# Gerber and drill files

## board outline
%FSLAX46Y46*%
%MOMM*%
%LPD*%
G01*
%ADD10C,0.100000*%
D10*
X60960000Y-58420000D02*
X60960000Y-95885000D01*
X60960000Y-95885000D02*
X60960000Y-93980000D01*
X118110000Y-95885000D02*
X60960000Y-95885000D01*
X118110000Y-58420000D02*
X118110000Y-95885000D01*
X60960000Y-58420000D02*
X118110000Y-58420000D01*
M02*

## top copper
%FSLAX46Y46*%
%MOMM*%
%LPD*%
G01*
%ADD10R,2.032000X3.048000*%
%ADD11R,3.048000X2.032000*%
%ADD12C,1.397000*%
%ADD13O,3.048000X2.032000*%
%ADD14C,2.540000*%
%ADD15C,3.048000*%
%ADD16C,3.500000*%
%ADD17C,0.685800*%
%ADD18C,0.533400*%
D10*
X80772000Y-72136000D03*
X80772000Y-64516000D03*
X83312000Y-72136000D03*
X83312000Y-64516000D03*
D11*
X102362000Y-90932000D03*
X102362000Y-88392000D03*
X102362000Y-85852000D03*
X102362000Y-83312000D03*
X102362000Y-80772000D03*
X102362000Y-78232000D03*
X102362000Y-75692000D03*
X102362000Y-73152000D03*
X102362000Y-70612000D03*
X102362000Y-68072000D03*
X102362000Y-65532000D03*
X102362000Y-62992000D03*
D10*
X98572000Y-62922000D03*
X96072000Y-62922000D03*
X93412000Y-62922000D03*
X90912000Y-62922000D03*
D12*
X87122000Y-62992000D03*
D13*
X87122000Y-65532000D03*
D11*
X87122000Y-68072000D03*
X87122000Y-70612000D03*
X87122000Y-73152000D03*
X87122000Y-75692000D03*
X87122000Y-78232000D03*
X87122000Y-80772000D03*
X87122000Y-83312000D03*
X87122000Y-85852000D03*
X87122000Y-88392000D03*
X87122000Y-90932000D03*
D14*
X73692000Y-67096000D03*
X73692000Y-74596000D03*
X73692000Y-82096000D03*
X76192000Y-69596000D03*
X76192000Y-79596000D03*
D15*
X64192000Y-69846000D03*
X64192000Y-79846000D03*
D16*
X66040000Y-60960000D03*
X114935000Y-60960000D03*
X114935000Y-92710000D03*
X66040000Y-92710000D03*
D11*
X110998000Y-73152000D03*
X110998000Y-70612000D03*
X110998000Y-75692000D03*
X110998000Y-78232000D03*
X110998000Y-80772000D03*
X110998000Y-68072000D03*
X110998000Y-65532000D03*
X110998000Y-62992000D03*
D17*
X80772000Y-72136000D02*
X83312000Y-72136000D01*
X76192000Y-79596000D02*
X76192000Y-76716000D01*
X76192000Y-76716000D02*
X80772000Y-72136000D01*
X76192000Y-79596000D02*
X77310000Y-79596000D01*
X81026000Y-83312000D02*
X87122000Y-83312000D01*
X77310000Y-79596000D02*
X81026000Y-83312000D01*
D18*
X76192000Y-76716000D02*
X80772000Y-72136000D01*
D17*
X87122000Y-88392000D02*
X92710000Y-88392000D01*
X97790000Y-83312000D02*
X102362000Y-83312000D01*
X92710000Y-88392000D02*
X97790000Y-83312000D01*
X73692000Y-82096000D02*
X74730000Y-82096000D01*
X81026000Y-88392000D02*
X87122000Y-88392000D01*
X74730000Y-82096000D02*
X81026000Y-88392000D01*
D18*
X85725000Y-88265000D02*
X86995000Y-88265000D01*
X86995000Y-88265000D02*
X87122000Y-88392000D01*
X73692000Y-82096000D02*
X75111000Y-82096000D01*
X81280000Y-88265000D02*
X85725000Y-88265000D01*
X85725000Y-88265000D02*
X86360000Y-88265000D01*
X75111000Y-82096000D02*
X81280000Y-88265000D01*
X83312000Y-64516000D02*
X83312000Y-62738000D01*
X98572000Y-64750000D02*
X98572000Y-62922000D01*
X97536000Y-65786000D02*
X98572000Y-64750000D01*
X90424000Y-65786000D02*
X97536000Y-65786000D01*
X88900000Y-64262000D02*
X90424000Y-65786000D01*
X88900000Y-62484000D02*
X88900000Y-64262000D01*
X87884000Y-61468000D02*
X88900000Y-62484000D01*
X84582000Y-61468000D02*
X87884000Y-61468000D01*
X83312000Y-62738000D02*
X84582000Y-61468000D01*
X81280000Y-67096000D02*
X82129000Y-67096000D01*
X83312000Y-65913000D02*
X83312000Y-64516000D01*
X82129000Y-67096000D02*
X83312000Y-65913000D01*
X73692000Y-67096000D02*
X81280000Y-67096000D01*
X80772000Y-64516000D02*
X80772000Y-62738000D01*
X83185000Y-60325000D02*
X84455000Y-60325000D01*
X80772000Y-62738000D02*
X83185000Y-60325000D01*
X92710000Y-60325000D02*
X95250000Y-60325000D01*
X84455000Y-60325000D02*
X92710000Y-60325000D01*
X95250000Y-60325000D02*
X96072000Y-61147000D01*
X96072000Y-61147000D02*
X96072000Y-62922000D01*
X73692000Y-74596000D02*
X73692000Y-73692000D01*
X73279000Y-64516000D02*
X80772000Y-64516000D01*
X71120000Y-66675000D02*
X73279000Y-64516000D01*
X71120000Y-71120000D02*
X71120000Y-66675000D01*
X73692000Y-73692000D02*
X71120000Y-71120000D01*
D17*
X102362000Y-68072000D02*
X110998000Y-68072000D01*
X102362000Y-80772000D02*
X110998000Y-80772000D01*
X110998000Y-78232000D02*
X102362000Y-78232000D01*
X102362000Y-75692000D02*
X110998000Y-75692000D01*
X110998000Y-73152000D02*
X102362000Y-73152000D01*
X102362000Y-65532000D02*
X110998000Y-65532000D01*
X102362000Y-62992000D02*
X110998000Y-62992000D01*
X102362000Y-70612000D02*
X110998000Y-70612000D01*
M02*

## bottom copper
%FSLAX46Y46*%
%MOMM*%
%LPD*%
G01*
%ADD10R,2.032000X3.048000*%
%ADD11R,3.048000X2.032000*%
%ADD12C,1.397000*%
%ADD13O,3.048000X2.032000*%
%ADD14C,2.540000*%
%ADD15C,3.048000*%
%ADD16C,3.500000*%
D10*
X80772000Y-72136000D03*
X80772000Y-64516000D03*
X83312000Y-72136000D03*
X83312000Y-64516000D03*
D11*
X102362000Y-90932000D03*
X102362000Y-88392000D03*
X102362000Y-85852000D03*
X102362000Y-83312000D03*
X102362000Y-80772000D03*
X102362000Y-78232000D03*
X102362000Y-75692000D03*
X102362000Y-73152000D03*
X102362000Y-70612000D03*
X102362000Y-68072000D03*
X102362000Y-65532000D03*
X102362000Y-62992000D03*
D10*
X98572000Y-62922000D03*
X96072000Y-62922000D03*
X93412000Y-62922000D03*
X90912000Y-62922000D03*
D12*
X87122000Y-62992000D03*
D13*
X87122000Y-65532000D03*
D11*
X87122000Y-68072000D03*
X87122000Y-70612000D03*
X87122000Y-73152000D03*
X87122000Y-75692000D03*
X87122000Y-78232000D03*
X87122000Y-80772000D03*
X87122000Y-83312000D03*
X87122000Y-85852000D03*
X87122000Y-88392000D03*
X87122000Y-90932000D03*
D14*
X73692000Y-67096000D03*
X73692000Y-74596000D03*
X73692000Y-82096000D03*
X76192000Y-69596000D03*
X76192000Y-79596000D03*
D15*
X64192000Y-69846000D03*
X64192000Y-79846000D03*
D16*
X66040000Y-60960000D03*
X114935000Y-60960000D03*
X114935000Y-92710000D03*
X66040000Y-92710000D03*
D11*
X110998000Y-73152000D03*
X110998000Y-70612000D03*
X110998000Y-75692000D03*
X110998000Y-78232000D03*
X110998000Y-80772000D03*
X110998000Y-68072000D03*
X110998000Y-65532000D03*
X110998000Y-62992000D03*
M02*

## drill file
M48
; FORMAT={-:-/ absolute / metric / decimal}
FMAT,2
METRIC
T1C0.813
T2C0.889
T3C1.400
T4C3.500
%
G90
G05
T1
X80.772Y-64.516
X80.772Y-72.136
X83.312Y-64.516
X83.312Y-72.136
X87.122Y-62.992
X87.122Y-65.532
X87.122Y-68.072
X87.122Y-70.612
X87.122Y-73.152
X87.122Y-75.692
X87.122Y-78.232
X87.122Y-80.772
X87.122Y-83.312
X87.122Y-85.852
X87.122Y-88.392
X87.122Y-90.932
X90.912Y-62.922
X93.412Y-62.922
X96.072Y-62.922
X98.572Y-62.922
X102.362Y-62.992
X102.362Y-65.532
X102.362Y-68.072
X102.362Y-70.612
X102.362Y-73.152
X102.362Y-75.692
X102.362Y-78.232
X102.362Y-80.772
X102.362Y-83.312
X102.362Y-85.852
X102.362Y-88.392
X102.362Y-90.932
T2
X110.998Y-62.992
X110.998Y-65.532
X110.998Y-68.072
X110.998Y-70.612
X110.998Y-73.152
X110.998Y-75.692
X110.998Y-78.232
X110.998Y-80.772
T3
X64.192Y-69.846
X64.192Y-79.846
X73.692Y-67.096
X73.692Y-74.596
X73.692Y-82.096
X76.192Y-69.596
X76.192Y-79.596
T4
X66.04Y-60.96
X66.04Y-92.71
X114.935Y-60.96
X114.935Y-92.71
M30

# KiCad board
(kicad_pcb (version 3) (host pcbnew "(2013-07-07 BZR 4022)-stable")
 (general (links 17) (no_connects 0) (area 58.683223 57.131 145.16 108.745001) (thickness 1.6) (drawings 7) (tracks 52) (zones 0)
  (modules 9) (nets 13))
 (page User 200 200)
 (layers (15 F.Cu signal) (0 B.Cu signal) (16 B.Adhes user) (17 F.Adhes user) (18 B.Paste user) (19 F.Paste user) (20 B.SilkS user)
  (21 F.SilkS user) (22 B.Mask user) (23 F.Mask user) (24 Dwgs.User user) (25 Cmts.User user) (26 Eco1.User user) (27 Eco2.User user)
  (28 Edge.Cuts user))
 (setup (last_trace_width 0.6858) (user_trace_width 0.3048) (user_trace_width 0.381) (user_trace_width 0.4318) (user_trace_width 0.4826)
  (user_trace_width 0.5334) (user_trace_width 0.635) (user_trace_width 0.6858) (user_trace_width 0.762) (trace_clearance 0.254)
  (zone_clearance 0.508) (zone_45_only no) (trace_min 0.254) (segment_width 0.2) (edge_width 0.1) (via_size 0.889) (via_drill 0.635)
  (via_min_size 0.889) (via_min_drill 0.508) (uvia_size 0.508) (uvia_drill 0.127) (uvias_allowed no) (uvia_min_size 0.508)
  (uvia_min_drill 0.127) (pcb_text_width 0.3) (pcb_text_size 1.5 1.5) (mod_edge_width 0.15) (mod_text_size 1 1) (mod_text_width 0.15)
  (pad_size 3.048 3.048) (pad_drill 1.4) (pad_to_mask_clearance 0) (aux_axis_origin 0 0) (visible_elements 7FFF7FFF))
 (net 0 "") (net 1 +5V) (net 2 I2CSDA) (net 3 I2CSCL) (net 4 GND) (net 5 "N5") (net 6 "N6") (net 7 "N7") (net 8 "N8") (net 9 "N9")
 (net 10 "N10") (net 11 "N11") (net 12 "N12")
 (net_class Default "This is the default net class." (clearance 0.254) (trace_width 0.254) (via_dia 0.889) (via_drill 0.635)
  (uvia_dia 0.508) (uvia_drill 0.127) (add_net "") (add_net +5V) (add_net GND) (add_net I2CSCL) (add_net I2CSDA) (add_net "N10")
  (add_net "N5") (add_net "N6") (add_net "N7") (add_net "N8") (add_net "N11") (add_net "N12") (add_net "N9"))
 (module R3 (layer F.Cu) (at 80.772 68.326 90) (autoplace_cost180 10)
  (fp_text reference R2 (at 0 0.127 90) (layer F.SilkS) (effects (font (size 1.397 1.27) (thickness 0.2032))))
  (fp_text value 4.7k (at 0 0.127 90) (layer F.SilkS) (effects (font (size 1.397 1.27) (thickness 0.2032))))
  (pad 1 thru_hole rect (at -3.81 0 90) (size 3.048 2.032) (drill 0.8128) (layers *.Cu *.Mask F.SilkS) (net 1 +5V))
  (pad 2 thru_hole rect (at 3.81 0 90) (size 3.048 2.032) (drill 0.8128) (layers *.Cu *.Mask F.SilkS) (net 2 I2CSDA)))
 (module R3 (layer F.Cu) (at 83.312 68.326 90) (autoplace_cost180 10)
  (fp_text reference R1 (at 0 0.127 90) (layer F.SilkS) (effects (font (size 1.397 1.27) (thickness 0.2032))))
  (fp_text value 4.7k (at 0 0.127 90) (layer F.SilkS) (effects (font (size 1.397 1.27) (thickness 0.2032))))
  (pad 1 thru_hole rect (at -3.81 0 90) (size 3.048 2.032) (drill 0.8128) (layers *.Cu *.Mask F.SilkS) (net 1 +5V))
  (pad 2 thru_hole rect (at 3.81 0 90) (size 3.048 2.032) (drill 0.8128) (layers *.Cu *.Mask F.SilkS) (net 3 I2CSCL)))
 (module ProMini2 (layer F.Cu) (at 94.742 74.422 90)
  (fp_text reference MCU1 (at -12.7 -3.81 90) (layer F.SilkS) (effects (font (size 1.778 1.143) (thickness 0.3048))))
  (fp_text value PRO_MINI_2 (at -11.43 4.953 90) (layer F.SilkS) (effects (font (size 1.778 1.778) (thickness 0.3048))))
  (pad 1 thru_hole rect (at -16.51 7.62 90) (size 2.032 3.048) (drill 0.8128) (layers *.Cu *.Mask F.SilkS))
  (pad 2 thru_hole rect (at -13.97 7.62 90) (size 2.032 3.048) (drill 0.8128) (layers *.Cu *.Mask F.SilkS))
  (pad 3 thru_hole rect (at -11.43 7.62 90) (size 2.032 3.048) (drill 0.8128) (layers *.Cu *.Mask F.SilkS))
  (pad 4 thru_hole rect (at -8.89 7.62 90) (size 2.032 3.048) (drill 0.8128) (layers *.Cu *.Mask F.SilkS) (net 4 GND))
  (pad 5 thru_hole rect (at -6.35 7.62 90) (size 2.032 3.048) (drill 0.8128) (layers *.Cu *.Mask F.SilkS) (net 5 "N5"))
  (pad 6 thru_hole rect (at -3.81 7.62 90) (size 2.032 3.048) (drill 0.8128) (layers *.Cu *.Mask F.SilkS) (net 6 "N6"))
  (pad 7 thru_hole rect (at -1.27 7.62 90) (size 2.032 3.048) (drill 0.8128) (layers *.Cu *.Mask F.SilkS) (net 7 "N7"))
  (pad 8 thru_hole rect (at 1.27 7.62 90) (size 2.032 3.048) (drill 0.8128) (layers *.Cu *.Mask F.SilkS) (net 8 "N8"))
  (pad 9 thru_hole rect (at 3.81 7.62 90) (size 2.032 3.048) (drill 0.8128) (layers *.Cu *.Mask F.SilkS) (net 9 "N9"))
  (pad 10 thru_hole rect (at 6.35 7.62 90) (size 2.032 3.048) (drill 0.8128) (layers *.Cu *.Mask F.SilkS) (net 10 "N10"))
  (pad 11 thru_hole rect (at 8.89 7.62 90) (size 2.032 3.048) (drill 0.8128) (layers *.Cu *.Mask F.SilkS) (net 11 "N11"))
  (pad 12 thru_hole rect (at 11.43 7.62 90) (size 2.032 3.048) (drill 0.8128) (layers *.Cu *.Mask F.SilkS) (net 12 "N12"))
  (pad 13 thru_hole rect (at 11.5 3.83 90) (size 3.048 2.032) (drill 0.8128) (layers *.Cu *.Mask F.SilkS) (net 3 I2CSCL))
  (pad 14 thru_hole rect (at 11.5 1.33 90) (size 3.048 2.032) (drill 0.8128) (layers *.Cu *.Mask F.SilkS) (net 2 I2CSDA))
  (pad 15 thru_hole rect (at 11.5 -1.33 90) (size 3.048 2.032) (drill 0.8128) (layers *.Cu *.Mask F.SilkS))
  (pad 16 thru_hole rect (at 11.5 -3.83 90) (size 3.048 2.032) (drill 0.8128) (layers *.Cu *.Mask F.SilkS))
  (pad 17 thru_hole circle (at 11.43 -7.62 90) (size 1.397 1.397) (drill 0.8128) (layers *.Cu *.Mask F.SilkS))
  (pad 18 thru_hole oval (at 8.89 -7.62 90) (size 2.032 3.048) (drill 0.8128) (layers *.Cu *.Mask F.SilkS))
  (pad 19 thru_hole rect (at 6.35 -7.62 90) (size 2.032 3.048) (drill 0.8128) (layers *.Cu *.Mask F.SilkS))
  (pad 20 thru_hole rect (at 3.81 -7.62 90) (size 2.032 3.048) (drill 0.8128) (layers *.Cu *.Mask F.SilkS))
  (pad 21 thru_hole rect (at 1.27 -7.62 90) (size 2.032 3.048) (drill 0.8128) (layers *.Cu *.Mask F.SilkS))
  (pad 22 thru_hole rect (at -1.27 -7.62 90) (size 2.032 3.048) (drill 0.8128) (layers *.Cu *.Mask F.SilkS))
  (pad 23 thru_hole rect (at -3.81 -7.62 90) (size 2.032 3.048) (drill 0.8128) (layers *.Cu *.Mask F.SilkS))
  (pad 24 thru_hole rect (at -6.35 -7.62 90) (size 2.032 3.048) (drill 0.8128) (layers *.Cu *.Mask F.SilkS))
  (pad 25 thru_hole rect (at -8.89 -7.62 90) (size 2.032 3.048) (drill 0.8128) (layers *.Cu *.Mask F.SilkS) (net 1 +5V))
  (pad 26 thru_hole rect (at -11.43 -7.62 90) (size 2.032 3.048) (drill 0.8128) (layers *.Cu *.Mask F.SilkS))
  (pad 27 thru_hole rect (at -13.97 -7.62 90) (size 2.032 3.048) (drill 0.8128) (layers *.Cu *.Mask F.SilkS) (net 4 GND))
  (pad 28 thru_hole rect (at -16.51 -7.62 90) (size 2.032 3.048) (drill 0.8128) (layers *.Cu *.Mask F.SilkS)))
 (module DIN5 (layer F.Cu) (at 75.692 69.596 270)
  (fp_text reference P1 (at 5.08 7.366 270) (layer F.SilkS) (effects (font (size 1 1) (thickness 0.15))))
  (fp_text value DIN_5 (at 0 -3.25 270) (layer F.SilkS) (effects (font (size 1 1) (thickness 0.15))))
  (pad 1 thru_hole circle (at -2.5 2 270) (size 2.54 2.54) (drill 1.4) (layers *.Cu *.Mask F.SilkS) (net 3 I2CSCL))
  (pad 2 thru_hole circle (at 5 2 270) (size 2.54 2.54) (drill 1.4) (layers *.Cu *.Mask F.SilkS) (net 2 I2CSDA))
  (pad 3 thru_hole circle (at 12.5 2 270) (size 2.54 2.54) (drill 1.4) (layers *.Cu *.Mask F.SilkS) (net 4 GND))
  (pad 5 thru_hole circle (at 0 -0.5 270) (size 2.54 2.54) (drill 1.4) (layers *.Cu *.Mask F.SilkS))
  (pad 4 thru_hole circle (at 10 -0.5 270) (size 2.54 2.54) (drill 1.4) (layers *.Cu *.Mask F.SilkS) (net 1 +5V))
  (pad "" thru_hole circle (at 0.25 11.5 270) (size 3.048 3.048) (drill 1.4) (layers *.Cu *.Mask F.SilkS))
  (pad "" thru_hole circle (at 10.25 11.5 270) (size 3.048 3.048) (drill 1.4) (layers *.Cu *.Mask F.SilkS)))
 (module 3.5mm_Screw (layer F.Cu) (at 66.04 60.96)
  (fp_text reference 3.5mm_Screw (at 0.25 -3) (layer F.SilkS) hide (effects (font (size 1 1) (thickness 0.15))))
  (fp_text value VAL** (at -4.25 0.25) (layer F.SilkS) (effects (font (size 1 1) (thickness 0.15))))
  (pad 1 thru_hole circle (at 0 0) (size 3.5 3.5) (drill 3.5) (layers *.Cu *.Mask F.SilkS)))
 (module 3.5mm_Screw (layer F.Cu) (at 114.935 60.96)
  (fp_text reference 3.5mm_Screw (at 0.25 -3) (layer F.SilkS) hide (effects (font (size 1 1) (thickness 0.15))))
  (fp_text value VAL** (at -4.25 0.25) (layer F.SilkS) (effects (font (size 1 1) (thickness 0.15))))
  (pad 1 thru_hole circle (at 0 0) (size 3.5 3.5) (drill 3.5) (layers *.Cu *.Mask F.SilkS)))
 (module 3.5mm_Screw (layer F.Cu) (at 114.935 92.71)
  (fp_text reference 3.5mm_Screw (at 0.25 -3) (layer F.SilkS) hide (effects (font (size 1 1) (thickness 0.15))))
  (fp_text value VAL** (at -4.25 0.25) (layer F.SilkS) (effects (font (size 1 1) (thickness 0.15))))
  (pad 1 thru_hole circle (at 0 0) (size 3.5 3.5) (drill 3.5) (layers *.Cu *.Mask F.SilkS)))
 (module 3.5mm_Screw (layer F.Cu) (at 66.04 92.71)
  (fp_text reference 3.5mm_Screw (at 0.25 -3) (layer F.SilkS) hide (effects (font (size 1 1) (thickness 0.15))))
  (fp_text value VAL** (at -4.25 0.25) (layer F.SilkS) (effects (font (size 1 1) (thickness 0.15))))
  (pad 1 thru_hole circle (at 0 0) (size 3.5 3.5) (drill 3.5) (layers *.Cu *.Mask F.SilkS)))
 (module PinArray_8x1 (layer F.Cu) (at 110.998 71.882 270)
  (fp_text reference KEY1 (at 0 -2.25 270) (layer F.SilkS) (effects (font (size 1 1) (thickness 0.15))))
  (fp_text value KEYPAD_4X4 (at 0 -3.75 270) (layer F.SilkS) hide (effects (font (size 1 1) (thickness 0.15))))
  (pad 5 thru_hole rect (at 1.27 0 270) (size 2.032 3.048) (drill 0.889) (layers *.Cu *.Mask F.SilkS) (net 8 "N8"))
  (pad 4 thru_hole rect (at -1.27 0 270) (size 2.032 3.048) (drill 0.889) (layers *.Cu *.Mask F.SilkS) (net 9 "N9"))
  (pad 6 thru_hole rect (at 3.81 0 270) (size 2.032 3.048) (drill 0.889) (layers *.Cu *.Mask F.SilkS) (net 7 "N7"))
  (pad 7 thru_hole rect (at 6.35 0 270) (size 2.032 3.048) (drill 0.889) (layers *.Cu *.Mask F.SilkS) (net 6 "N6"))
  (pad 8 thru_hole rect (at 8.89 0 270) (size 2.032 3.048) (drill 0.889) (layers *.Cu *.Mask F.SilkS) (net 5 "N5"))
  (pad 3 thru_hole rect (at -3.81 0 270) (size 2.032 3.048) (drill 0.889) (layers *.Cu *.Mask F.SilkS) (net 10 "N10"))
  (pad 2 thru_hole rect (at -6.35 0 270) (size 2.032 3.048) (drill 0.889) (layers *.Cu *.Mask F.SilkS) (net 11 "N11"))
  (pad 1 thru_hole rect (at -8.89 0 270) (size 2.032 3.048) (drill 0.889) (layers *.Cu *.Mask F.SilkS) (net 12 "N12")))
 (gr_line (start 60.96 58.42) (end 60.96 95.885) (angle 90) (layer Edge.Cuts) (width 0.1))
 (gr_line (start 60.96 95.885) (end 60.96 93.98) (angle 90) (layer Edge.Cuts) (width 0.1))
 (gr_line (start 118.11 95.885) (end 60.96 95.885) (angle 90) (layer Edge.Cuts) (width 0.1))
 (gr_line (start 118.11 58.42) (end 118.11 95.885) (angle 90) (layer Edge.Cuts) (width 0.1))
 (gr_line (start 60.96 58.42) (end 118.11 58.42) (angle 90) (layer Edge.Cuts) (width 0.1))
 (segment (start 80.772 72.136) (end 83.312 72.136) (width 0.6858) (layer F.Cu) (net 1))
 (segment (start 76.192 79.596) (end 76.192 76.716) (width 0.6858) (layer F.Cu) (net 1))
 (segment (start 76.192 76.716) (end 80.772 72.136) (width 0.6858) (layer F.Cu) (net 1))
 (segment (start 76.192 79.596) (end 77.31 79.596) (width 0.6858) (layer F.Cu) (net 1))
 (segment (start 81.026 83.312) (end 87.122 83.312) (width 0.6858) (layer F.Cu) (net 1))
 (segment (start 77.31 79.596) (end 81.026 83.312) (width 0.6858) (layer F.Cu) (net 1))
 (segment (start 76.192 76.716) (end 80.772 72.136) (width 0.5334) (layer F.Cu) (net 1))
 (segment (start 87.122 88.392) (end 92.71 88.392) (width 0.6858) (layer F.Cu) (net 4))
 (segment (start 97.79 83.312) (end 102.362 83.312) (width 0.6858) (layer F.Cu) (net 4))
 (segment (start 92.71 88.392) (end 97.79 83.312) (width 0.6858) (layer F.Cu) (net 4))
 (segment (start 73.692 82.096) (end 74.73 82.096) (width 0.6858) (layer F.Cu) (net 4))
 (segment (start 81.026 88.392) (end 87.122 88.392) (width 0.6858) (layer F.Cu) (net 4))
 (segment (start 74.73 82.096) (end 81.026 88.392) (width 0.6858) (layer F.Cu) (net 4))
 (segment (start 85.725 88.265) (end 86.995 88.265) (width 0.5334) (layer F.Cu) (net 4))
 (segment (start 86.995 88.265) (end 87.122 88.392) (width 0.5334) (layer F.Cu) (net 4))
 (segment (start 73.692 82.096) (end 75.111 82.096) (width 0.5334) (layer F.Cu) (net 4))
 (segment (start 81.28 88.265) (end 85.725 88.265) (width 0.5334) (layer F.Cu) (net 4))
 (segment (start 85.725 88.265) (end 86.36 88.265) (width 0.5334) (layer F.Cu) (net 4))
 (segment (start 75.111 82.096) (end 81.28 88.265) (width 0.5334) (layer F.Cu) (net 4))
 (segment (start 83.312 64.516) (end 83.312 62.738) (width 0.5334) (layer F.Cu) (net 3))
 (segment (start 98.572 64.75) (end 98.572 62.922) (width 0.5334) (layer F.Cu) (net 3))
 (segment (start 97.536 65.786) (end 98.572 64.75) (width 0.5334) (layer F.Cu) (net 3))
 (segment (start 90.424 65.786) (end 97.536 65.786) (width 0.5334) (layer F.Cu) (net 3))
 (segment (start 88.9 64.262) (end 90.424 65.786) (width 0.5334) (layer F.Cu) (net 3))
 (segment (start 88.9 62.484) (end 88.9 64.262) (width 0.5334) (layer F.Cu) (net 3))
 (segment (start 87.884 61.468) (end 88.9 62.484) (width 0.5334) (layer F.Cu) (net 3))
 (segment (start 84.582 61.468) (end 87.884 61.468) (width 0.5334) (layer F.Cu) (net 3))
 (segment (start 83.312 62.738) (end 84.582 61.468) (width 0.5334) (layer F.Cu) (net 3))
 (segment (start 81.28 67.096) (end 82.129 67.096) (width 0.5334) (layer F.Cu) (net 3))
 (segment (start 83.312 65.913) (end 83.312 64.516) (width 0.5334) (layer F.Cu) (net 3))
 (segment (start 82.129 67.096) (end 83.312 65.913) (width 0.5334) (layer F.Cu) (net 3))
 (segment (start 73.692 67.096) (end 81.28 67.096) (width 0.5334) (layer F.Cu) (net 3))
 (segment (start 80.772 64.516) (end 80.772 62.738) (width 0.5334) (layer F.Cu) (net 2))
 (segment (start 83.185 60.325) (end 84.455 60.325) (width 0.5334) (layer F.Cu) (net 2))
 (segment (start 80.772 62.738) (end 83.185 60.325) (width 0.5334) (layer F.Cu) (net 2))
 (segment (start 92.71 60.325) (end 95.25 60.325) (width 0.5334) (layer F.Cu) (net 2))
 (segment (start 84.455 60.325) (end 92.71 60.325) (width 0.5334) (layer F.Cu) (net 2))
 (segment (start 95.25 60.325) (end 96.072 61.147) (width 0.5334) (layer F.Cu) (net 2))
 (segment (start 96.072 61.147) (end 96.072 62.922) (width 0.5334) (layer F.Cu) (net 2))
 (segment (start 73.692 74.596) (end 73.692 73.692) (width 0.5334) (layer F.Cu) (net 2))
 (segment (start 73.279 64.516) (end 80.772 64.516) (width 0.5334) (layer F.Cu) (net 2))
 (segment (start 71.12 66.675) (end 73.279 64.516) (width 0.5334) (layer F.Cu) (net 2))
 (segment (start 71.12 71.12) (end 71.12 66.675) (width 0.5334) (layer F.Cu) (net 2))
 (segment (start 73.692 73.692) (end 71.12 71.12) (width 0.5334) (layer F.Cu) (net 2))
 (segment (start 102.362 68.072) (end 110.998 68.072) (width 0.6858) (layer F.Cu) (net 10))
 (segment (start 102.362 80.772) (end 110.998 80.772) (width 0.6858) (layer F.Cu) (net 5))
 (segment (start 110.998 78.232) (end 102.362 78.232) (width 0.6858) (layer F.Cu) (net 6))
 (segment (start 102.362 75.692) (end 110.998 75.692) (width 0.6858) (layer F.Cu) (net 7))
 (segment (start 110.998 73.152) (end 102.362 73.152) (width 0.6858) (layer F.Cu) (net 8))
 (segment (start 102.362 65.532) (end 110.998 65.532) (width 0.6858) (layer F.Cu) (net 11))
 (segment (start 102.362 62.992) (end 110.998 62.992) (width 0.6858) (layer F.Cu) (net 12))
 (segment (start 102.362 70.612) (end 110.998 70.612) (width 0.6858) (layer F.Cu) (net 9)))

